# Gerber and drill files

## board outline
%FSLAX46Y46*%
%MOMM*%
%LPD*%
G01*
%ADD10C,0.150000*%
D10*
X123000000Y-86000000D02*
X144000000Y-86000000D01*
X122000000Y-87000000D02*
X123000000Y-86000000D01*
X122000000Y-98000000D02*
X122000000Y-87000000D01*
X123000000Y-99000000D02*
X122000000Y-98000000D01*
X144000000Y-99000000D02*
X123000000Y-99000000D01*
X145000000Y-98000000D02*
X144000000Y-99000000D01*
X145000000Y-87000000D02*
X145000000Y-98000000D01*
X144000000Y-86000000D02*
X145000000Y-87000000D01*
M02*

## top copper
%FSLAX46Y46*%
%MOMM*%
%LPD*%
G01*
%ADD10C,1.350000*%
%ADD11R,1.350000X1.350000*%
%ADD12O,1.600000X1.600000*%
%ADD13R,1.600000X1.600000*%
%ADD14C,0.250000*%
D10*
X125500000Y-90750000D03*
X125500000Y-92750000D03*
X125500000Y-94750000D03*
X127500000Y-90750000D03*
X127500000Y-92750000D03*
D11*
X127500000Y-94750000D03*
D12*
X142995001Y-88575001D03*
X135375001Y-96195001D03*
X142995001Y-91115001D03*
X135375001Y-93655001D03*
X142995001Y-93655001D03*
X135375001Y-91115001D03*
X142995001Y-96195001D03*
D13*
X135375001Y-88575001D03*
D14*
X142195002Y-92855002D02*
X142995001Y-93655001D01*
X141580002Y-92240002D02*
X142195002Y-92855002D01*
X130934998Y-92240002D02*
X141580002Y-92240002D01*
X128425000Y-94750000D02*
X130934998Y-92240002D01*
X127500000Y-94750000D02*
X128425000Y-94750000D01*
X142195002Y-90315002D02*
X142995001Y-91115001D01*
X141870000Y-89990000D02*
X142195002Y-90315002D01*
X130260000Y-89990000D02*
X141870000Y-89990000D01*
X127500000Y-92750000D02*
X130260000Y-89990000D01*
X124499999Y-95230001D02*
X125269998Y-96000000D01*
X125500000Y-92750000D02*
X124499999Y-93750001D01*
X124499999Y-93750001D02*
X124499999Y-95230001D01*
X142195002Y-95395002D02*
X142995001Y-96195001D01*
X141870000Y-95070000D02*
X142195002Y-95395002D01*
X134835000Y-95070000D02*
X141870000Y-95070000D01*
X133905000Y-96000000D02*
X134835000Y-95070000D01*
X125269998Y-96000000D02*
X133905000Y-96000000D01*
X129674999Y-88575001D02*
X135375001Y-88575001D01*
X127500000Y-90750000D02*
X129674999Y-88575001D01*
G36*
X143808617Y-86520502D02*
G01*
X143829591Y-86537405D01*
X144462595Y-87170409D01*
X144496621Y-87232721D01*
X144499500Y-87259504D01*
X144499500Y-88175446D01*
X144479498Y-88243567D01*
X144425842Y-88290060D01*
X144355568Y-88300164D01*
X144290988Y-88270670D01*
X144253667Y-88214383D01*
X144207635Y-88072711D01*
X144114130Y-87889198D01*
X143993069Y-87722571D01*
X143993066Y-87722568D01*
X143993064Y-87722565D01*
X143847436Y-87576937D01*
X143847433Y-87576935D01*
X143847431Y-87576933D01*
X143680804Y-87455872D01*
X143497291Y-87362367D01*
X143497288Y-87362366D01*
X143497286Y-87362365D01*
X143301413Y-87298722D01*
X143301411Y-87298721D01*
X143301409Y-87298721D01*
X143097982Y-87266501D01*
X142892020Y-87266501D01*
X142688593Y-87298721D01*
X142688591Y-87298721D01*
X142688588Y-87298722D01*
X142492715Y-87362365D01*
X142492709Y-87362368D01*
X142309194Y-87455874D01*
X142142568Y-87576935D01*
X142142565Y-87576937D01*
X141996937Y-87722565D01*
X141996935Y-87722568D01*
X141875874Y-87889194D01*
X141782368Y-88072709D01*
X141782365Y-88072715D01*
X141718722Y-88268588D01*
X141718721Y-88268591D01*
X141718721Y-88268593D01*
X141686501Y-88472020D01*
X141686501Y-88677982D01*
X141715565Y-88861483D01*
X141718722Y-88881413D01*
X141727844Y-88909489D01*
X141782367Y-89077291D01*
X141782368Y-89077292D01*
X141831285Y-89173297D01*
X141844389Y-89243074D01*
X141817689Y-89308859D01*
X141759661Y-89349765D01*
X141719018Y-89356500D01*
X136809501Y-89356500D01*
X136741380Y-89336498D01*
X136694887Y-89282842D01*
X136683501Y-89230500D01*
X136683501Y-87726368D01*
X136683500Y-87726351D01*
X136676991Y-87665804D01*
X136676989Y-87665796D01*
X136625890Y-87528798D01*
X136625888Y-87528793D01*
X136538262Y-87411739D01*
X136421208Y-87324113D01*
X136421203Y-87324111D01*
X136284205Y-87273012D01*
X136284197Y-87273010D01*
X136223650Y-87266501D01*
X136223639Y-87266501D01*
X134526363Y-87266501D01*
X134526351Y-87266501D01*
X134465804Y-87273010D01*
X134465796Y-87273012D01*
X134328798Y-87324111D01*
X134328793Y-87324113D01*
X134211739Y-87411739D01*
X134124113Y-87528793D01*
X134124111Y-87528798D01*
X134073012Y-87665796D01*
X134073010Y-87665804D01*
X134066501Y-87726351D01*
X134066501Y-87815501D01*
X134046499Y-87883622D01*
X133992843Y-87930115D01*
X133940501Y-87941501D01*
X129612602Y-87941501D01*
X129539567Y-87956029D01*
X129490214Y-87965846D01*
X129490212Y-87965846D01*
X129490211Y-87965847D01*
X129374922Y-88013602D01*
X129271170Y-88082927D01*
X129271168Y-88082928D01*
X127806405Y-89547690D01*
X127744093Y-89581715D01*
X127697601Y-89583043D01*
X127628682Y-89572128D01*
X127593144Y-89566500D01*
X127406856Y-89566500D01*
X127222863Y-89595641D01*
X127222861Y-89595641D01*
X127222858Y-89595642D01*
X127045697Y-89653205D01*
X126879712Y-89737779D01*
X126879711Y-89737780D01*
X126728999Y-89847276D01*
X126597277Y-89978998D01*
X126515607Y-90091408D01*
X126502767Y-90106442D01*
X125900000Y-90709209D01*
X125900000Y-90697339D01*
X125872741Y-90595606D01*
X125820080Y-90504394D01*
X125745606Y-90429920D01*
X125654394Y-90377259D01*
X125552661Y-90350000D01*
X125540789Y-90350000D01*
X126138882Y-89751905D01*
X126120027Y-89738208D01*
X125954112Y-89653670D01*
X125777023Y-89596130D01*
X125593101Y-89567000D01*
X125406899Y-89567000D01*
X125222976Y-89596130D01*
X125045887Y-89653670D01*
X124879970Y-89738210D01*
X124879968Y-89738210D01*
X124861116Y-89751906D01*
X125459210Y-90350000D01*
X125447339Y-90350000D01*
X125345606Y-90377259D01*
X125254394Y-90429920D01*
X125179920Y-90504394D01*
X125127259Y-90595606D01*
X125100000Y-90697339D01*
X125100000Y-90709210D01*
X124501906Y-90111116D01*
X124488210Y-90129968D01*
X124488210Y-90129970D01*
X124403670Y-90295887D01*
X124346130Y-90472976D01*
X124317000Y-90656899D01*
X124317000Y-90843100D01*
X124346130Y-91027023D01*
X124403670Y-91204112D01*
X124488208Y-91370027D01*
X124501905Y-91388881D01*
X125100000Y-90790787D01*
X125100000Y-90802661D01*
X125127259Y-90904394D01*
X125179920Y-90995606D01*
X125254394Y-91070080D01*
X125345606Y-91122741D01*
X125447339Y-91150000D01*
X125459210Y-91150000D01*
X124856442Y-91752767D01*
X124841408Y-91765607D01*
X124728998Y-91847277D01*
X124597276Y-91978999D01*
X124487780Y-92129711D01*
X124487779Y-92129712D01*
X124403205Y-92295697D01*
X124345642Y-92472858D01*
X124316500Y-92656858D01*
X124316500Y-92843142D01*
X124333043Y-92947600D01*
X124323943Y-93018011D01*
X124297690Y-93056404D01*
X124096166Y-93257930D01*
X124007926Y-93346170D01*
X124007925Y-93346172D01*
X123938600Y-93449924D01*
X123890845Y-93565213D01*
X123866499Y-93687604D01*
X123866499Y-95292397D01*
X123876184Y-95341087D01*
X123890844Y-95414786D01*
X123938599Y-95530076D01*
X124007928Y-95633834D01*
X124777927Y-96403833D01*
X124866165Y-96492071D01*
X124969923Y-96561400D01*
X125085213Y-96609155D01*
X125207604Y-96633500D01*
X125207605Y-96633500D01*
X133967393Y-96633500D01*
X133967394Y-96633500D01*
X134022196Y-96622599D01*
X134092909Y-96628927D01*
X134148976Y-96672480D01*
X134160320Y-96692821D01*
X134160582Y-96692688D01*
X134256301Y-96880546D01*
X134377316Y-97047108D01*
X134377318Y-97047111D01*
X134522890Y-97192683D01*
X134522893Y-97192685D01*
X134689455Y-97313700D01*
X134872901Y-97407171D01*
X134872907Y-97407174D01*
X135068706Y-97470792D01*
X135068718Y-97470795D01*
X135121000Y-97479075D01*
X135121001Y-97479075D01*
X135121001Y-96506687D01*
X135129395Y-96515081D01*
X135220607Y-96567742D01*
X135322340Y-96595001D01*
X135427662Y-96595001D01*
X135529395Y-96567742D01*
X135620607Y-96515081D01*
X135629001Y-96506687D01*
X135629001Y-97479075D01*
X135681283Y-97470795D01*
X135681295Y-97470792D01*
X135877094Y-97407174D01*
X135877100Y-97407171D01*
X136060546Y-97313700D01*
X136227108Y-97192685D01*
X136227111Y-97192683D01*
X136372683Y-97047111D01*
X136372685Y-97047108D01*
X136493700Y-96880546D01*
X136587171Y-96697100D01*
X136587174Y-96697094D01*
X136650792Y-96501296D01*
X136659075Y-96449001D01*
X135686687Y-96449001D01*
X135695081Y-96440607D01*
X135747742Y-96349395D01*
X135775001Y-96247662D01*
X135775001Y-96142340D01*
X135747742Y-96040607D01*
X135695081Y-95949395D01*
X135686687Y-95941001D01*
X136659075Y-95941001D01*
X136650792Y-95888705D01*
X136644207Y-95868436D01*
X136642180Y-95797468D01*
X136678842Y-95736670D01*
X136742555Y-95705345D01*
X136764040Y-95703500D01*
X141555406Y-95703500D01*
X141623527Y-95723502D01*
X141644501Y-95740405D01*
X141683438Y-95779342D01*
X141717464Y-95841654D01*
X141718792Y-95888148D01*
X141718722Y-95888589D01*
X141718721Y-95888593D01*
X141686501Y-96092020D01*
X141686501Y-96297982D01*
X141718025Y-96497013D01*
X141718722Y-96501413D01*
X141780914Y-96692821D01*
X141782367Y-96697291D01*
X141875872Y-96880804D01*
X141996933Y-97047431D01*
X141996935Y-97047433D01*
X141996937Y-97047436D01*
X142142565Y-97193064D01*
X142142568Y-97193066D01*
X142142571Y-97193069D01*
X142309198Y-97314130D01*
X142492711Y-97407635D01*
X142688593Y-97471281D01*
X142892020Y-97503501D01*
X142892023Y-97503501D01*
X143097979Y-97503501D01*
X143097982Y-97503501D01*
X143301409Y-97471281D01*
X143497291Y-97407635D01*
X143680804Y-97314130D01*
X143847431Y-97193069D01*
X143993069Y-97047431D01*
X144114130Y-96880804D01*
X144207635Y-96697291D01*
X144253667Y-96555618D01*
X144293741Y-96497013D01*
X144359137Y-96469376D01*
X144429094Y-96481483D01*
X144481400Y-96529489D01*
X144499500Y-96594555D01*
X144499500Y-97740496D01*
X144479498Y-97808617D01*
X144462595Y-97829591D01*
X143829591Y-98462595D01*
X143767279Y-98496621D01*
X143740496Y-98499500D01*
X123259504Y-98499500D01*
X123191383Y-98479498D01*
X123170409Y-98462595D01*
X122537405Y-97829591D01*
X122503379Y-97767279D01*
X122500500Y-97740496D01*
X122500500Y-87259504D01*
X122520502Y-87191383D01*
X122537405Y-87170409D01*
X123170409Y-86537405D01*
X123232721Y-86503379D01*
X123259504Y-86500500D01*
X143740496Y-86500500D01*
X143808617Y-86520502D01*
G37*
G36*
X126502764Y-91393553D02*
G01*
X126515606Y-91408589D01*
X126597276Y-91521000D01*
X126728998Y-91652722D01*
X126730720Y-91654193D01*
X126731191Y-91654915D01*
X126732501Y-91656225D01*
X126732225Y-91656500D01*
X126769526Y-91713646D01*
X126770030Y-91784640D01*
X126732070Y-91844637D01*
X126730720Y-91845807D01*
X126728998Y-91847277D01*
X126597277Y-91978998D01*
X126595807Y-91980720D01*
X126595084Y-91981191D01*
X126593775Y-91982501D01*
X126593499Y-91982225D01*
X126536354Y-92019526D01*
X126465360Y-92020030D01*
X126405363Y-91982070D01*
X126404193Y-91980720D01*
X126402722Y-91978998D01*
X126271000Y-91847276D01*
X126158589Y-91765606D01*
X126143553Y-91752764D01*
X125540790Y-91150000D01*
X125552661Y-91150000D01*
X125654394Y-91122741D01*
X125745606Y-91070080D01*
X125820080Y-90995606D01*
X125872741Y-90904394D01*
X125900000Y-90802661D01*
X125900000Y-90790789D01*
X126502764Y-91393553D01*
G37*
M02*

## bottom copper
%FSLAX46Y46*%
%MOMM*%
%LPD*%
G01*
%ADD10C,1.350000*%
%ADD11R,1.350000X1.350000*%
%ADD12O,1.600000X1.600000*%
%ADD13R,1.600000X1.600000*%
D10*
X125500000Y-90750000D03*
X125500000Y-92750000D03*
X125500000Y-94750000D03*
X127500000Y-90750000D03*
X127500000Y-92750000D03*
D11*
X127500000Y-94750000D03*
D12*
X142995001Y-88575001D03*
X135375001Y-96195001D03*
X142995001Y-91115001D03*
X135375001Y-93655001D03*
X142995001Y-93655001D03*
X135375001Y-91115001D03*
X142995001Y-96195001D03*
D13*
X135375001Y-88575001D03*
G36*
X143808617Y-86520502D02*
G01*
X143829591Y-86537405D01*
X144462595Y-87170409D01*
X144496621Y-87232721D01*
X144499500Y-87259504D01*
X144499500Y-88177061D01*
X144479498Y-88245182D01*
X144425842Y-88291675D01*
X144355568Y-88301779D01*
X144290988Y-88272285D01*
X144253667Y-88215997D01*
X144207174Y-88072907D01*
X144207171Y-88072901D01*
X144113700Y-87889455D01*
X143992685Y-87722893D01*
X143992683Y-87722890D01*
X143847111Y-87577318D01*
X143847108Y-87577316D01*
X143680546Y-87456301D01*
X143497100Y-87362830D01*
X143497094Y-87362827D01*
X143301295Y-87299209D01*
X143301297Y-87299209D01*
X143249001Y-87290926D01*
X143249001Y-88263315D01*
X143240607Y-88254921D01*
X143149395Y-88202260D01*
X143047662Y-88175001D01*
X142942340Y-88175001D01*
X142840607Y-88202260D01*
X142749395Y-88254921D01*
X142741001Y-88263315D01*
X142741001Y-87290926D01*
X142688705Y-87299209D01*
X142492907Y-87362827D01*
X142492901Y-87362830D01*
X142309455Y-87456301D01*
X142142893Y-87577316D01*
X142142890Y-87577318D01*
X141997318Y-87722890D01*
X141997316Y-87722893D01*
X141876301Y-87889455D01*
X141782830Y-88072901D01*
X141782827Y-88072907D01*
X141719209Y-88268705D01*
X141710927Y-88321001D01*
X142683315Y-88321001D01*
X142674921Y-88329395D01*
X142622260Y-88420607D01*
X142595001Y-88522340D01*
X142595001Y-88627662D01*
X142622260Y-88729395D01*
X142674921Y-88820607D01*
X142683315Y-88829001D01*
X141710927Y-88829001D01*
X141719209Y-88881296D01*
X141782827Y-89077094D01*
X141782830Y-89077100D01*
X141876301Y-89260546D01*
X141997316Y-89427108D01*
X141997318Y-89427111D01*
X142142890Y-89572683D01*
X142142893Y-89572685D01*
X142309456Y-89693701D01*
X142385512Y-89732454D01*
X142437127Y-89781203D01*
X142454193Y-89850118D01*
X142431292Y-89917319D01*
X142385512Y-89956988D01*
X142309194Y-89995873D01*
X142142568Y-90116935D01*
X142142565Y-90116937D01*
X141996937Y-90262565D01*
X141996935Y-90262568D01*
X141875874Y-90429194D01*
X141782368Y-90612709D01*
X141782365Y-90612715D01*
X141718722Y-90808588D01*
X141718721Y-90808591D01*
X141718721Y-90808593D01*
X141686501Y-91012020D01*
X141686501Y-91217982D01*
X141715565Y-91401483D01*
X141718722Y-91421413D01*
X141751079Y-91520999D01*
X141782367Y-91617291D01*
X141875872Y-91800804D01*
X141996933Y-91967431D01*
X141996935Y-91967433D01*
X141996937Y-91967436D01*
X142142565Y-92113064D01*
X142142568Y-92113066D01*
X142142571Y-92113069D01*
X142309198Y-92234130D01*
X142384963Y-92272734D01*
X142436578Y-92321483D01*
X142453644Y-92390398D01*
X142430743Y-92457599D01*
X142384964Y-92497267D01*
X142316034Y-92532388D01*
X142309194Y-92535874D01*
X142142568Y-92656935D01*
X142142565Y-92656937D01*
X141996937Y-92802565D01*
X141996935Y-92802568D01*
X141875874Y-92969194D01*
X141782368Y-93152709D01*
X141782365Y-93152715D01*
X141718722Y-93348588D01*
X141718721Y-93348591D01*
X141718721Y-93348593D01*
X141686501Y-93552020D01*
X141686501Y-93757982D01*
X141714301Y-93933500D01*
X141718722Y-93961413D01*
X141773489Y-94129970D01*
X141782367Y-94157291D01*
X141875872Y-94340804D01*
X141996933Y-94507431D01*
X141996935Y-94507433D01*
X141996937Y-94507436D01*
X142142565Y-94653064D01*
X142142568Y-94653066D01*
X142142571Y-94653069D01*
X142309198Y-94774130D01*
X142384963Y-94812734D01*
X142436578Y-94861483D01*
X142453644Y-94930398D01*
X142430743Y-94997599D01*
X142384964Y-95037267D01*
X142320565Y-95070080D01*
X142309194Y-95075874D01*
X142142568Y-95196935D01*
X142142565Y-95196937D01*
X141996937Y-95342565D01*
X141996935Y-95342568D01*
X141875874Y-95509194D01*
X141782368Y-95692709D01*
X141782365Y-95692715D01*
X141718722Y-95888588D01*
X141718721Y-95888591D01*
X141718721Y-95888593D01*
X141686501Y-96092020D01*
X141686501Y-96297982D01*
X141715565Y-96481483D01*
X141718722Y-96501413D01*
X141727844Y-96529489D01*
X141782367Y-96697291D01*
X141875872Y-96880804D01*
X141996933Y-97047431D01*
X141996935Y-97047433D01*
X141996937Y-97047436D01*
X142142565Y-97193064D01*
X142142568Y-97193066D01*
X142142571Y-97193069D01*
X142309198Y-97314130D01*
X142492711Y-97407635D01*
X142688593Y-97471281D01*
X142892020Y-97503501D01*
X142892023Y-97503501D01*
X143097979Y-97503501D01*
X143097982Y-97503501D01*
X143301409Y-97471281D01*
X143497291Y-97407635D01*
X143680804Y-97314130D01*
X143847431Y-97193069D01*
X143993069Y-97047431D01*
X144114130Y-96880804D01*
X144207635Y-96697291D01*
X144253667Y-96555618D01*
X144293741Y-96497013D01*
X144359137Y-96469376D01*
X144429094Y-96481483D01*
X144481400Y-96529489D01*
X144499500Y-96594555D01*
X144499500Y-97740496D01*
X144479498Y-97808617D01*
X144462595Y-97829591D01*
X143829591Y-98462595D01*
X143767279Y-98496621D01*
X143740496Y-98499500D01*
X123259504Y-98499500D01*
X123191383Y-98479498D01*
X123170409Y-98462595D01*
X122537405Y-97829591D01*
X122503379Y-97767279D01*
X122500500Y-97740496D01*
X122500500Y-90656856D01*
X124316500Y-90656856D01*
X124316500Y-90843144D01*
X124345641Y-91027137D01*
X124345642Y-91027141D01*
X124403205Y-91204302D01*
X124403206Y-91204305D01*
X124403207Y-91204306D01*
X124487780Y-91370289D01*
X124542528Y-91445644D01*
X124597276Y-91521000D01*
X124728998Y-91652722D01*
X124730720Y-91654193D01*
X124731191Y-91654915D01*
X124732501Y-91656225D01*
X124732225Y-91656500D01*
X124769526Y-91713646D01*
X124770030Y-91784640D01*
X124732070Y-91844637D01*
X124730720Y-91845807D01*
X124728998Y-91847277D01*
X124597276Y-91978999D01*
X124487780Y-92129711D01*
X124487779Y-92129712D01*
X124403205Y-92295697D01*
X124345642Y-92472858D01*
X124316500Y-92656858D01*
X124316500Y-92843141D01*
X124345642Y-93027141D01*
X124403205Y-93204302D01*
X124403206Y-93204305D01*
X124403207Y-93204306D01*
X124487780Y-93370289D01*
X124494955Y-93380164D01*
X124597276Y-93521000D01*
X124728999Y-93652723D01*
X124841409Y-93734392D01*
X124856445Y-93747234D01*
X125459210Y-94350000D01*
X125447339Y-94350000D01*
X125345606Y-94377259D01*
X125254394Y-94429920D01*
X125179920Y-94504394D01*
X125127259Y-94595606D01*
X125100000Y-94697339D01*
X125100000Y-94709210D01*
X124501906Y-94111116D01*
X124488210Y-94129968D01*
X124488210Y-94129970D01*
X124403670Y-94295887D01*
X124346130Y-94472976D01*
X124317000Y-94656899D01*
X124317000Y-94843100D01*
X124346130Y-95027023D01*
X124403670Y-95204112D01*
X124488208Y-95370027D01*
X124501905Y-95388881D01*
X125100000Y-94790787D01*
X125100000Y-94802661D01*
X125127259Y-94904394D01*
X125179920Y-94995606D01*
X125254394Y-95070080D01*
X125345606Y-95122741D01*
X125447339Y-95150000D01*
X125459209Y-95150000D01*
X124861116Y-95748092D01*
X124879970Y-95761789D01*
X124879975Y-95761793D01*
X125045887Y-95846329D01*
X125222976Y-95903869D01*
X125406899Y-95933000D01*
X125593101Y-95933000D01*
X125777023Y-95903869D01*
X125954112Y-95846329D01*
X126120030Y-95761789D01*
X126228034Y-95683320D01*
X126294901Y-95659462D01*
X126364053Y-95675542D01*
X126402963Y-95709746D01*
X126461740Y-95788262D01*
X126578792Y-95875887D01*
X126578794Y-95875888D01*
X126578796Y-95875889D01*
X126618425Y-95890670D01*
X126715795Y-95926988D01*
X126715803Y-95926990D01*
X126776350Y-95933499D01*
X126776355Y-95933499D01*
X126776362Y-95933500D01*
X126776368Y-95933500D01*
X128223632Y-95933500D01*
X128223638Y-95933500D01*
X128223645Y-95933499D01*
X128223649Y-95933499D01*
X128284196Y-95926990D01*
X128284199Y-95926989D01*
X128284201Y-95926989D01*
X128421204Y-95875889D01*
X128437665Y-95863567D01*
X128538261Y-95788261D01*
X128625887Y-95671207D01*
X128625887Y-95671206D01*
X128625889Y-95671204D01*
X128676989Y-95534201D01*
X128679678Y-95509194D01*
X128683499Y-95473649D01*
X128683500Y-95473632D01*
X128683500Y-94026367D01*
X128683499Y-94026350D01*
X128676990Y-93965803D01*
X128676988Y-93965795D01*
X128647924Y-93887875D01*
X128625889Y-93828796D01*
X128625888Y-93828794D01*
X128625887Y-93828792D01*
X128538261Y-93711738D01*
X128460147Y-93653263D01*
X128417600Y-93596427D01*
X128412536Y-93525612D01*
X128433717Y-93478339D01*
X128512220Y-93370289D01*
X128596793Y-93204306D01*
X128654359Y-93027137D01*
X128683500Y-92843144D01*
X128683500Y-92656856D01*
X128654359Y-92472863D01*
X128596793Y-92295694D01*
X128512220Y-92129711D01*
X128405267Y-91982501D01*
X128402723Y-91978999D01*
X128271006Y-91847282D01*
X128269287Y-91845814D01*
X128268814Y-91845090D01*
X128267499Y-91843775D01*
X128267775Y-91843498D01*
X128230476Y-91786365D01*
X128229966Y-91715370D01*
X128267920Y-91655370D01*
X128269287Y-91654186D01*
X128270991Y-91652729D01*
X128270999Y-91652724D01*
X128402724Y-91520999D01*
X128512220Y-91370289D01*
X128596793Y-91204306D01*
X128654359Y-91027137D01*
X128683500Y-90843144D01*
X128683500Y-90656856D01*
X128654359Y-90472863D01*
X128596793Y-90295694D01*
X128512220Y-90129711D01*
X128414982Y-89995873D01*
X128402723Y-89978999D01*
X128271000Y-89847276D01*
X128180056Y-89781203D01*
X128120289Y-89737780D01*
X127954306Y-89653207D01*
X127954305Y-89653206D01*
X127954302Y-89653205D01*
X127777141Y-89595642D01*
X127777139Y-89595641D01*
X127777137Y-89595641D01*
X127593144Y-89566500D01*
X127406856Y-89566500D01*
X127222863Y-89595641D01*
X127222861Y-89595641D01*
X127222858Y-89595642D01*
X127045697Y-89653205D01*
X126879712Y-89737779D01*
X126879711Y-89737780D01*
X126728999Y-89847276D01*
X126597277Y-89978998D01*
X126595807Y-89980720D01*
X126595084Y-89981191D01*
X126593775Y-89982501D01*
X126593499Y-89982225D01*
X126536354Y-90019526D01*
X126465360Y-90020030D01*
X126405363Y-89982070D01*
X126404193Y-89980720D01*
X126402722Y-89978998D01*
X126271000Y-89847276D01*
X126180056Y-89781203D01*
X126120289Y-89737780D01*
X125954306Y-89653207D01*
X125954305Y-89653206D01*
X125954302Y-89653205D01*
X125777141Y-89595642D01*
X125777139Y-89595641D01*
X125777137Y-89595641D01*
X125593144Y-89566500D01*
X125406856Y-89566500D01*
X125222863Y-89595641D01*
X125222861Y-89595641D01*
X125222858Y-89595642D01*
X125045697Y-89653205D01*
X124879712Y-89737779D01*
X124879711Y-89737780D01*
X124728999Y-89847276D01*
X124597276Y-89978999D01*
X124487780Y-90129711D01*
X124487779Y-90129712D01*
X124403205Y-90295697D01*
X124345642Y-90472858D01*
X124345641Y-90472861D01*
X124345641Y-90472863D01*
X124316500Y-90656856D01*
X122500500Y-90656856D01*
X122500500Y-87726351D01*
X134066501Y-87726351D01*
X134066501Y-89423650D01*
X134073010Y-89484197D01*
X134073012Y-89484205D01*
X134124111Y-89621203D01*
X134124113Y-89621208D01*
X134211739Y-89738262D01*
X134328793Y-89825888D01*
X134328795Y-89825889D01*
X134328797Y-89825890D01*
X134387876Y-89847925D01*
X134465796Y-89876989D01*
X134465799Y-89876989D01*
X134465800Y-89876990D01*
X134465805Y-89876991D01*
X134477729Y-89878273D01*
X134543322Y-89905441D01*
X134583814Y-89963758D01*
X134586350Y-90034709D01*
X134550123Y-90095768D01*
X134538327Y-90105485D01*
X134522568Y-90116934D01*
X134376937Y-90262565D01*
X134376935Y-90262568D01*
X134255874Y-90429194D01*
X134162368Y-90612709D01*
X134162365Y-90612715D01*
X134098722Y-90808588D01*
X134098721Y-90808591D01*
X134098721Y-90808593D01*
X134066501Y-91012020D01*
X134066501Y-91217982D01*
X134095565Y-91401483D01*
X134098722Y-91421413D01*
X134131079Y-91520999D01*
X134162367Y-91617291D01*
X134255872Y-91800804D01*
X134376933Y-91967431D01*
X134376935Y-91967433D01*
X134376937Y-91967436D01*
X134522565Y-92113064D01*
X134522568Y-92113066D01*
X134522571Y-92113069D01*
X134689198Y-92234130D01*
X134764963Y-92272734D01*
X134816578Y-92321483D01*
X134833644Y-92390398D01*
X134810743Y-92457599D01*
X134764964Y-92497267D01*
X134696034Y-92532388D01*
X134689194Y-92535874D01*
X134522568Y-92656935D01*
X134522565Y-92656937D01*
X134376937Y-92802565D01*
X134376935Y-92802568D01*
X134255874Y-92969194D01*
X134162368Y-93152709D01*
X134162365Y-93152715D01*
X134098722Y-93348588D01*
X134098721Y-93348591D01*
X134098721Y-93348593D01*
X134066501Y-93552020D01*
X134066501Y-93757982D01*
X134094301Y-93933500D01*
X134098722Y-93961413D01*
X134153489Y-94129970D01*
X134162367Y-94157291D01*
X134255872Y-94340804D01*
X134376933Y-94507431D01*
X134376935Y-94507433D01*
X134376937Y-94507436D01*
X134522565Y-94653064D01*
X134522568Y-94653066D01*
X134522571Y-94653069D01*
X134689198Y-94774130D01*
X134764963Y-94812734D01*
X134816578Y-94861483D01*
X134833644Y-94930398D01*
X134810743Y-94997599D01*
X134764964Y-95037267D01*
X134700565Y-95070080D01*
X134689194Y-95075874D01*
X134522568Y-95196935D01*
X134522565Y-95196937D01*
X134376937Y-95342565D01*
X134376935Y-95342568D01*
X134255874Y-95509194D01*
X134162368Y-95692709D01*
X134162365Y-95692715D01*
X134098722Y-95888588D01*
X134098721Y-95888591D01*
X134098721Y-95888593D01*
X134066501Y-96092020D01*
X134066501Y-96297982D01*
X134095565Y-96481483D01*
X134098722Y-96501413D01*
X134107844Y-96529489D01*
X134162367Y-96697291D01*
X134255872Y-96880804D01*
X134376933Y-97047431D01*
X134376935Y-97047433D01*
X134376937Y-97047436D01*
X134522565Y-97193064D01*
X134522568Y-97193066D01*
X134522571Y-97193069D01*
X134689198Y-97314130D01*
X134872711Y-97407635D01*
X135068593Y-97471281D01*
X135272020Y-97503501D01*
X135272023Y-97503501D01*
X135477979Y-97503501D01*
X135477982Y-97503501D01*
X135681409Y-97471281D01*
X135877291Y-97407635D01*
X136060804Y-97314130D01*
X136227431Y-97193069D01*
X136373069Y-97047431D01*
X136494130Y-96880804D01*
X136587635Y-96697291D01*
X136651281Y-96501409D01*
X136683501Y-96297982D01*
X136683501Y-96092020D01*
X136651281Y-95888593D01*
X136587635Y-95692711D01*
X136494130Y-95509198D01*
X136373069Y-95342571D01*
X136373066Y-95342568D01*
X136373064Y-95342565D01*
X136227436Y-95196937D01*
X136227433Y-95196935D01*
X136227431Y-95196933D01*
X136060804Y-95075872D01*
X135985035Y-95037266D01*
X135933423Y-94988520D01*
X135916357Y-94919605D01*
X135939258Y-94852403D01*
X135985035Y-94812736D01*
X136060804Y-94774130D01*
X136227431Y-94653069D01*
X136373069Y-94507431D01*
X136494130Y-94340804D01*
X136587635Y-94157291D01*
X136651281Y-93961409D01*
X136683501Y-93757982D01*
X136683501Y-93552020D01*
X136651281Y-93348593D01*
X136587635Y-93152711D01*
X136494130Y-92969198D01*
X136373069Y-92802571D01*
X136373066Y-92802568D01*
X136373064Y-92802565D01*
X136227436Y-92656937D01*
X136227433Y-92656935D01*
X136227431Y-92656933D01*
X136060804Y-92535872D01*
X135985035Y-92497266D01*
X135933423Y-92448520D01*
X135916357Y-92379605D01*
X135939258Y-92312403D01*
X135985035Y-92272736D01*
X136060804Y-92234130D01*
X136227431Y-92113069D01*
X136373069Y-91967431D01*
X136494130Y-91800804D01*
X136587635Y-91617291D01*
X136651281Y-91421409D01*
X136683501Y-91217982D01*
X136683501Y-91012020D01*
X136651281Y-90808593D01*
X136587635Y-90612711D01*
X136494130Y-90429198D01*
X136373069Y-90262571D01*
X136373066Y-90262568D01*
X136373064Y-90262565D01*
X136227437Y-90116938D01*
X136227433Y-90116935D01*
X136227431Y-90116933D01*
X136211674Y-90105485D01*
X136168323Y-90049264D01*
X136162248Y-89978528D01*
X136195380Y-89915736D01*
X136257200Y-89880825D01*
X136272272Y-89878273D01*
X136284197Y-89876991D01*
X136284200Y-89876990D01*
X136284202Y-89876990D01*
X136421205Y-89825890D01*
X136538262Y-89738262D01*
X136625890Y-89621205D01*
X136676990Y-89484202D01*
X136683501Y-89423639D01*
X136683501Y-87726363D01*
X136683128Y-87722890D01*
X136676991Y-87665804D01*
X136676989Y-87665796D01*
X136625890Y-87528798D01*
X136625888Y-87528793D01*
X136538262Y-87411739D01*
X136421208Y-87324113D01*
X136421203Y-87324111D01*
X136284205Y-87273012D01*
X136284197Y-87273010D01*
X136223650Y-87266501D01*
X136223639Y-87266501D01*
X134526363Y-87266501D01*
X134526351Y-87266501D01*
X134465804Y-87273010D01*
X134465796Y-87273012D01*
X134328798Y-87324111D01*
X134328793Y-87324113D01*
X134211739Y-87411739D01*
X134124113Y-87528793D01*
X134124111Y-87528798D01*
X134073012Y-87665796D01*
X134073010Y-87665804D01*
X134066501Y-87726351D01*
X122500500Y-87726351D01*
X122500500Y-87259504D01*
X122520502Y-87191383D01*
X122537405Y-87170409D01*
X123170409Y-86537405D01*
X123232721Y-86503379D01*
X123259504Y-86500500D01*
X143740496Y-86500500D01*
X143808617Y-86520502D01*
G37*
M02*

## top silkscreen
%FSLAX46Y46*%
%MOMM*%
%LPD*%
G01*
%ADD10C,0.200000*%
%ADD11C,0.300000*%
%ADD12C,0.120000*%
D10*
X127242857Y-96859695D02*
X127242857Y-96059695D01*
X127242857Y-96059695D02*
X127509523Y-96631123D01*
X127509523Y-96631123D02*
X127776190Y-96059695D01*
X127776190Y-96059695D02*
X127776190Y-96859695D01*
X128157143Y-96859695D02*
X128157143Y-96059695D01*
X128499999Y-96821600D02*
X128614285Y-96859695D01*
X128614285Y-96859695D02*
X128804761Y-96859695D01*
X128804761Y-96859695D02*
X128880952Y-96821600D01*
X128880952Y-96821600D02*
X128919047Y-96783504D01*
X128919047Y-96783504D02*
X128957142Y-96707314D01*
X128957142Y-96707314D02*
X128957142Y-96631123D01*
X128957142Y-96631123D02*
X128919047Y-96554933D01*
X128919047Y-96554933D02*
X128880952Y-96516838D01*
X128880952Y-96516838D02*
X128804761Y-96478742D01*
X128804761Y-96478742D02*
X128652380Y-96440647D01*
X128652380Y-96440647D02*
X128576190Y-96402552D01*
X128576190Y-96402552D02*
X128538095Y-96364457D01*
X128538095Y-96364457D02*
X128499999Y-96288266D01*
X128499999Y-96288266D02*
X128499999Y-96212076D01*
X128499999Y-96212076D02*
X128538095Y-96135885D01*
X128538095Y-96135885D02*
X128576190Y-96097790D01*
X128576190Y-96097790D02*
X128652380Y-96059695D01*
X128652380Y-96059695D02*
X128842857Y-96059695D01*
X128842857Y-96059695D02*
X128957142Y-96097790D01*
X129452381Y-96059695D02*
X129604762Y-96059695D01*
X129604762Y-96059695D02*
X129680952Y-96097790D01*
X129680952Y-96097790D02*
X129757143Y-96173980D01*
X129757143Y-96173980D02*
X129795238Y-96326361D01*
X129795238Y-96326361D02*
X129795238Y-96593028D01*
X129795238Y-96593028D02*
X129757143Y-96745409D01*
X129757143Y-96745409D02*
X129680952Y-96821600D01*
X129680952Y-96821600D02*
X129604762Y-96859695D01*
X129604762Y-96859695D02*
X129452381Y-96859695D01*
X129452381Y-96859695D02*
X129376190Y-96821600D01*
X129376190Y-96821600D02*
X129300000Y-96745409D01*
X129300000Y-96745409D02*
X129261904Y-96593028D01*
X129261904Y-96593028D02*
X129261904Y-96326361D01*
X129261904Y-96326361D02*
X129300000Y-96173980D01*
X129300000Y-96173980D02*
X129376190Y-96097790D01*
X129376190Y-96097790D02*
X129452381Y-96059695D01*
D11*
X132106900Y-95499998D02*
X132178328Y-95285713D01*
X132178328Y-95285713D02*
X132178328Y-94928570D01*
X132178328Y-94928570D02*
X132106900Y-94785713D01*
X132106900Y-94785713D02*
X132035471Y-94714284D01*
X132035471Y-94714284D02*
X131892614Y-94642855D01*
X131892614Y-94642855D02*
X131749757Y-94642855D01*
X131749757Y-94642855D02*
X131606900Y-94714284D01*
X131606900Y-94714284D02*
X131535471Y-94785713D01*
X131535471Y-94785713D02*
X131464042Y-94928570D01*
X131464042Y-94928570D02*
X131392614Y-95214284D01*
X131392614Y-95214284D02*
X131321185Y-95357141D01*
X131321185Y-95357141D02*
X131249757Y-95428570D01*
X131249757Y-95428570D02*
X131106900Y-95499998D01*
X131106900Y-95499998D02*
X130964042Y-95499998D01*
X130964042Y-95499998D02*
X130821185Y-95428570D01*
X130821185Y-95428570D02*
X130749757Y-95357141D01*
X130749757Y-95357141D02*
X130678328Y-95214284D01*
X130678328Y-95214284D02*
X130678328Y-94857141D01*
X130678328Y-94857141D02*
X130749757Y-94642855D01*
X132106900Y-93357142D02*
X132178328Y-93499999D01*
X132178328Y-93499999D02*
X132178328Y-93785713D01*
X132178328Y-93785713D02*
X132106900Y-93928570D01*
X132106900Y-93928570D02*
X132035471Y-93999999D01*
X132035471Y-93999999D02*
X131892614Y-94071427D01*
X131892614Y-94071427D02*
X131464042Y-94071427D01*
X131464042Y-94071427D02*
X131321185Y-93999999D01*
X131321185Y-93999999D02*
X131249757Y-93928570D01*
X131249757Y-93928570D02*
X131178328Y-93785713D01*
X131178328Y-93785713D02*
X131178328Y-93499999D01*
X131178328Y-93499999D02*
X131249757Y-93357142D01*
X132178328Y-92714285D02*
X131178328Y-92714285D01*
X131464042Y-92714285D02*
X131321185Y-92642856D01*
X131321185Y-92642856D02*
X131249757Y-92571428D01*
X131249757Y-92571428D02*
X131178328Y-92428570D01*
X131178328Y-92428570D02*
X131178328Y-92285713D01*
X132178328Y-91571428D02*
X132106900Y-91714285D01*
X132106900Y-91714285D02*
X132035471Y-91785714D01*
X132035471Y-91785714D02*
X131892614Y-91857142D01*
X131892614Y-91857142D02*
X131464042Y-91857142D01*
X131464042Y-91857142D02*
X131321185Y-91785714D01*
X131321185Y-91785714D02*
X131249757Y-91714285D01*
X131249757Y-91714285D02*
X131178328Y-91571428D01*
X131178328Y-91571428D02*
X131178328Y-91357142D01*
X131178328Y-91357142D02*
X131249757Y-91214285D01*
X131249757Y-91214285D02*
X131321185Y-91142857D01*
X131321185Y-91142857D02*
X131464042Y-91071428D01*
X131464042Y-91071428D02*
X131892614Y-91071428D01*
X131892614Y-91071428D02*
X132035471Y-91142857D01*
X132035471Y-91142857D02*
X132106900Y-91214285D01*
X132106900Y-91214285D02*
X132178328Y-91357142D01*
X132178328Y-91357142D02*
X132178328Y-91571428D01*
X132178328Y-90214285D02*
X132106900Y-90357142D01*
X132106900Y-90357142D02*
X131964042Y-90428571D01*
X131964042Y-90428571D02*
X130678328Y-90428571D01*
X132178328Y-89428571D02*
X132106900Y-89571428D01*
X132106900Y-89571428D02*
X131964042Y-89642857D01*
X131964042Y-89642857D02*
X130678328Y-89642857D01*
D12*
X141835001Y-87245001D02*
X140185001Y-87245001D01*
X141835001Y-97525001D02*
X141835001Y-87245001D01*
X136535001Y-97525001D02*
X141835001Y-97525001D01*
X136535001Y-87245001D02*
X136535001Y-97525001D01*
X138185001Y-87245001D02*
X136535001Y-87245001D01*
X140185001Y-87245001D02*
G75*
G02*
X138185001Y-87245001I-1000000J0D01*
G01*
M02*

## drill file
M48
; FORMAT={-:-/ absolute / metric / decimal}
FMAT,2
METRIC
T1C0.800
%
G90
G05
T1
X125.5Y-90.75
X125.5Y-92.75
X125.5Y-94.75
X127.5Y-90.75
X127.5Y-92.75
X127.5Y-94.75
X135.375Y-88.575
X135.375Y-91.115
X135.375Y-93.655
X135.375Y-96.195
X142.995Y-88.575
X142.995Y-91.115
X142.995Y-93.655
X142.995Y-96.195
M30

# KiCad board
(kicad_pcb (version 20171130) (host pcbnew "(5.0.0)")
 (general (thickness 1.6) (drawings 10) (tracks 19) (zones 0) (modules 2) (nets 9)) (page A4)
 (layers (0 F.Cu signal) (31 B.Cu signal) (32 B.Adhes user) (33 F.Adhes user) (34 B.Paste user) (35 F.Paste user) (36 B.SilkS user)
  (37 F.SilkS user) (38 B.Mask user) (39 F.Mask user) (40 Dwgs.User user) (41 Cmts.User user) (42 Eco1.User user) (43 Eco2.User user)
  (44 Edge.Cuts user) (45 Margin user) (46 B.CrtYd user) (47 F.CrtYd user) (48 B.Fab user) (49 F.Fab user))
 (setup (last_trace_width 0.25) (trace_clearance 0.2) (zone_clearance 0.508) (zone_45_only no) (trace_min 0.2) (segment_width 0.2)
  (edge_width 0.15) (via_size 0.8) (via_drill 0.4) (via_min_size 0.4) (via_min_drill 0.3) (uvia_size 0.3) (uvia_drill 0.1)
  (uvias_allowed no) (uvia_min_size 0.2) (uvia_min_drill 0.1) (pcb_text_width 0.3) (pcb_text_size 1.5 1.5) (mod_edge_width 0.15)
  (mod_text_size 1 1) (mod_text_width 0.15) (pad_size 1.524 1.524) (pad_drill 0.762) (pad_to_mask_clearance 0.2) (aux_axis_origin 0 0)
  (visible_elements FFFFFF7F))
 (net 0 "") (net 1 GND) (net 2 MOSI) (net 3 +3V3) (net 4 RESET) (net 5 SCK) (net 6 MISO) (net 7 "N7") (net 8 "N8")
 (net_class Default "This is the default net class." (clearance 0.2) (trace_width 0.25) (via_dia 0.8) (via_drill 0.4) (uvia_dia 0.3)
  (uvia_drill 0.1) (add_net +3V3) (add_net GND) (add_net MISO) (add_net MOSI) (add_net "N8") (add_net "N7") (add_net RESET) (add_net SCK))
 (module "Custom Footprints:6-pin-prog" (layer F.Cu) (at 127.5 94.75 90)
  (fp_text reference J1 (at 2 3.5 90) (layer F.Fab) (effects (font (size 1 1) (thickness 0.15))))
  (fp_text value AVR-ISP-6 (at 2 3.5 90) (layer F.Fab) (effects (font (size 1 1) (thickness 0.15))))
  (pad 6 thru_hole circle (at 4 -2 90) (size 1.35 1.35) (drill 0.8) (layers *.Cu *.Mask) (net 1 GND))
  (pad 4 thru_hole circle (at 2 -2 90) (size 1.35 1.35) (drill 0.8) (layers *.Cu *.Mask) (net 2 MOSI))
  (pad 2 thru_hole circle (at 0 -2 90) (size 1.35 1.35) (drill 0.8) (layers *.Cu *.Mask) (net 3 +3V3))
  (pad 5 thru_hole circle (at 4 0 90) (size 1.35 1.35) (drill 0.8) (layers *.Cu *.Mask) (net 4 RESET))
  (pad 3 thru_hole circle (at 2 0 90) (size 1.35 1.35) (drill 0.8) (layers *.Cu *.Mask) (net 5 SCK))
  (pad 1 thru_hole rect (at 0 0 90) (size 1.35 1.35) (drill 0.8) (layers *.Cu *.Mask) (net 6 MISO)))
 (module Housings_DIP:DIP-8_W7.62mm (layer F.Cu) (at 135.375001 88.575001)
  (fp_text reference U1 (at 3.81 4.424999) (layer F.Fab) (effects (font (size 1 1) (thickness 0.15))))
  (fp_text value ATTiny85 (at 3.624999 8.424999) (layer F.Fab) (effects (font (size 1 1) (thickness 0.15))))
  (fp_line (start 6.46 -1.33) (end 4.81 -1.33) (layer F.SilkS) (width 0.12))
  (fp_line (start 6.46 8.95) (end 6.46 -1.33) (layer F.SilkS) (width 0.12))
  (fp_line (start 1.16 8.95) (end 6.46 8.95) (layer F.SilkS) (width 0.12))
  (fp_line (start 1.16 -1.33) (end 1.16 8.95) (layer F.SilkS) (width 0.12))
  (fp_line (start 2.81 -1.33) (end 1.16 -1.33) (layer F.SilkS) (width 0.12))
  (fp_arc (start 3.81 -1.33) (end 2.81 -1.33) (angle -180) (layer F.SilkS) (width 0.12))
  (pad 8 thru_hole oval (at 7.62 0) (size 1.6 1.6) (drill 0.8) (layers *.Cu *.Mask) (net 3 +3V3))
  (pad 4 thru_hole oval (at 0 7.62) (size 1.6 1.6) (drill 0.8) (layers *.Cu *.Mask) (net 1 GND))
  (pad 7 thru_hole oval (at 7.62 2.54) (size 1.6 1.6) (drill 0.8) (layers *.Cu *.Mask) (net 5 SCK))
  (pad 3 thru_hole oval (at 0 5.08) (size 1.6 1.6) (drill 0.8) (layers *.Cu *.Mask) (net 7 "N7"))
  (pad 6 thru_hole oval (at 7.62 5.08) (size 1.6 1.6) (drill 0.8) (layers *.Cu *.Mask) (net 6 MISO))
  (pad 2 thru_hole oval (at 0 2.54) (size 1.6 1.6) (drill 0.8) (layers *.Cu *.Mask) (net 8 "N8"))
  (pad 5 thru_hole oval (at 7.62 7.62) (size 1.6 1.6) (drill 0.8) (layers *.Cu *.Mask) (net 2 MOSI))
  (pad 1 thru_hole rect (at 0 0) (size 1.6 1.6) (drill 0.8) (layers *.Cu *.Mask) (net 4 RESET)))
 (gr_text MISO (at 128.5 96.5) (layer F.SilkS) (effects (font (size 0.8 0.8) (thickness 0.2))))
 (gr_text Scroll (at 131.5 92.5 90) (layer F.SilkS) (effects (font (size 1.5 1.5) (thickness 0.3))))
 (gr_line (start 123 86) (end 144 86) (layer Edge.Cuts) (width 0.15))
 (gr_line (start 122 87) (end 123 86) (layer Edge.Cuts) (width 0.15))
 (gr_line (start 122 98) (end 122 87) (layer Edge.Cuts) (width 0.15))
 (gr_line (start 123 99) (end 122 98) (layer Edge.Cuts) (width 0.15))
 (gr_line (start 144 99) (end 123 99) (layer Edge.Cuts) (width 0.15))
 (gr_line (start 145 98) (end 144 99) (layer Edge.Cuts) (width 0.15))
 (gr_line (start 145 87) (end 145 98) (layer Edge.Cuts) (width 0.15))
 (gr_line (start 144 86) (end 145 87) (layer Edge.Cuts) (width 0.15))
 (segment (start 142.195002 92.855002) (end 142.995001 93.655001) (width 0.25) (layer F.Cu) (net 6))
 (segment (start 141.580002 92.240002) (end 142.195002 92.855002) (width 0.25) (layer F.Cu) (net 6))
 (segment (start 130.934998 92.240002) (end 141.580002 92.240002) (width 0.25) (layer F.Cu) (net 6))
 (segment (start 128.425 94.75) (end 130.934998 92.240002) (width 0.25) (layer F.Cu) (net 6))
 (segment (start 127.5 94.75) (end 128.425 94.75) (width 0.25) (layer F.Cu) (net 6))
 (segment (start 142.195002 90.315002) (end 142.995001 91.115001) (width 0.25) (layer F.Cu) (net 5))
 (segment (start 141.87 89.99) (end 142.195002 90.315002) (width 0.25) (layer F.Cu) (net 5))
 (segment (start 130.26 89.99) (end 141.87 89.99) (width 0.25) (layer F.Cu) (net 5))
 (segment (start 127.5 92.75) (end 130.26 89.99) (width 0.25) (layer F.Cu) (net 5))
 (segment (start 124.499999 95.230001) (end 125.269998 96) (width 0.25) (layer F.Cu) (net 2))
 (segment (start 125.5 92.75) (end 124.499999 93.750001) (width 0.25) (layer F.Cu) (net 2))
 (segment (start 124.499999 93.750001) (end 124.499999 95.230001) (width 0.25) (layer F.Cu) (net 2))
 (segment (start 142.195002 95.395002) (end 142.995001 96.195001) (width 0.25) (layer F.Cu) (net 2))
 (segment (start 141.87 95.07) (end 142.195002 95.395002) (width 0.25) (layer F.Cu) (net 2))
 (segment (start 134.835 95.07) (end 141.87 95.07) (width 0.25) (layer F.Cu) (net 2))
 (segment (start 133.905 96) (end 134.835 95.07) (width 0.25) (layer F.Cu) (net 2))
 (segment (start 125.269998 96) (end 133.905 96) (width 0.25) (layer F.Cu) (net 2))
 (segment (start 129.674999 88.575001) (end 135.375001 88.575001) (width 0.25) (layer F.Cu) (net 4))
 (segment (start 127.5 90.75) (end 129.674999 88.575001) (width 0.25) (layer F.Cu) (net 4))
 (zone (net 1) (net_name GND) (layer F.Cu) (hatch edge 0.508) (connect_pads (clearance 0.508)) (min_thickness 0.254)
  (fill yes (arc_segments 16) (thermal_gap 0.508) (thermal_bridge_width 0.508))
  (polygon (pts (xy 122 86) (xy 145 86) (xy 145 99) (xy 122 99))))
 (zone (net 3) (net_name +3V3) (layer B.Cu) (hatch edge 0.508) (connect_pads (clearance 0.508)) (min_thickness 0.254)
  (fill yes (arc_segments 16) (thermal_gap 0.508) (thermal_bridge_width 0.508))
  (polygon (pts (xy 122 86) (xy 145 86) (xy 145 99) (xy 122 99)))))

